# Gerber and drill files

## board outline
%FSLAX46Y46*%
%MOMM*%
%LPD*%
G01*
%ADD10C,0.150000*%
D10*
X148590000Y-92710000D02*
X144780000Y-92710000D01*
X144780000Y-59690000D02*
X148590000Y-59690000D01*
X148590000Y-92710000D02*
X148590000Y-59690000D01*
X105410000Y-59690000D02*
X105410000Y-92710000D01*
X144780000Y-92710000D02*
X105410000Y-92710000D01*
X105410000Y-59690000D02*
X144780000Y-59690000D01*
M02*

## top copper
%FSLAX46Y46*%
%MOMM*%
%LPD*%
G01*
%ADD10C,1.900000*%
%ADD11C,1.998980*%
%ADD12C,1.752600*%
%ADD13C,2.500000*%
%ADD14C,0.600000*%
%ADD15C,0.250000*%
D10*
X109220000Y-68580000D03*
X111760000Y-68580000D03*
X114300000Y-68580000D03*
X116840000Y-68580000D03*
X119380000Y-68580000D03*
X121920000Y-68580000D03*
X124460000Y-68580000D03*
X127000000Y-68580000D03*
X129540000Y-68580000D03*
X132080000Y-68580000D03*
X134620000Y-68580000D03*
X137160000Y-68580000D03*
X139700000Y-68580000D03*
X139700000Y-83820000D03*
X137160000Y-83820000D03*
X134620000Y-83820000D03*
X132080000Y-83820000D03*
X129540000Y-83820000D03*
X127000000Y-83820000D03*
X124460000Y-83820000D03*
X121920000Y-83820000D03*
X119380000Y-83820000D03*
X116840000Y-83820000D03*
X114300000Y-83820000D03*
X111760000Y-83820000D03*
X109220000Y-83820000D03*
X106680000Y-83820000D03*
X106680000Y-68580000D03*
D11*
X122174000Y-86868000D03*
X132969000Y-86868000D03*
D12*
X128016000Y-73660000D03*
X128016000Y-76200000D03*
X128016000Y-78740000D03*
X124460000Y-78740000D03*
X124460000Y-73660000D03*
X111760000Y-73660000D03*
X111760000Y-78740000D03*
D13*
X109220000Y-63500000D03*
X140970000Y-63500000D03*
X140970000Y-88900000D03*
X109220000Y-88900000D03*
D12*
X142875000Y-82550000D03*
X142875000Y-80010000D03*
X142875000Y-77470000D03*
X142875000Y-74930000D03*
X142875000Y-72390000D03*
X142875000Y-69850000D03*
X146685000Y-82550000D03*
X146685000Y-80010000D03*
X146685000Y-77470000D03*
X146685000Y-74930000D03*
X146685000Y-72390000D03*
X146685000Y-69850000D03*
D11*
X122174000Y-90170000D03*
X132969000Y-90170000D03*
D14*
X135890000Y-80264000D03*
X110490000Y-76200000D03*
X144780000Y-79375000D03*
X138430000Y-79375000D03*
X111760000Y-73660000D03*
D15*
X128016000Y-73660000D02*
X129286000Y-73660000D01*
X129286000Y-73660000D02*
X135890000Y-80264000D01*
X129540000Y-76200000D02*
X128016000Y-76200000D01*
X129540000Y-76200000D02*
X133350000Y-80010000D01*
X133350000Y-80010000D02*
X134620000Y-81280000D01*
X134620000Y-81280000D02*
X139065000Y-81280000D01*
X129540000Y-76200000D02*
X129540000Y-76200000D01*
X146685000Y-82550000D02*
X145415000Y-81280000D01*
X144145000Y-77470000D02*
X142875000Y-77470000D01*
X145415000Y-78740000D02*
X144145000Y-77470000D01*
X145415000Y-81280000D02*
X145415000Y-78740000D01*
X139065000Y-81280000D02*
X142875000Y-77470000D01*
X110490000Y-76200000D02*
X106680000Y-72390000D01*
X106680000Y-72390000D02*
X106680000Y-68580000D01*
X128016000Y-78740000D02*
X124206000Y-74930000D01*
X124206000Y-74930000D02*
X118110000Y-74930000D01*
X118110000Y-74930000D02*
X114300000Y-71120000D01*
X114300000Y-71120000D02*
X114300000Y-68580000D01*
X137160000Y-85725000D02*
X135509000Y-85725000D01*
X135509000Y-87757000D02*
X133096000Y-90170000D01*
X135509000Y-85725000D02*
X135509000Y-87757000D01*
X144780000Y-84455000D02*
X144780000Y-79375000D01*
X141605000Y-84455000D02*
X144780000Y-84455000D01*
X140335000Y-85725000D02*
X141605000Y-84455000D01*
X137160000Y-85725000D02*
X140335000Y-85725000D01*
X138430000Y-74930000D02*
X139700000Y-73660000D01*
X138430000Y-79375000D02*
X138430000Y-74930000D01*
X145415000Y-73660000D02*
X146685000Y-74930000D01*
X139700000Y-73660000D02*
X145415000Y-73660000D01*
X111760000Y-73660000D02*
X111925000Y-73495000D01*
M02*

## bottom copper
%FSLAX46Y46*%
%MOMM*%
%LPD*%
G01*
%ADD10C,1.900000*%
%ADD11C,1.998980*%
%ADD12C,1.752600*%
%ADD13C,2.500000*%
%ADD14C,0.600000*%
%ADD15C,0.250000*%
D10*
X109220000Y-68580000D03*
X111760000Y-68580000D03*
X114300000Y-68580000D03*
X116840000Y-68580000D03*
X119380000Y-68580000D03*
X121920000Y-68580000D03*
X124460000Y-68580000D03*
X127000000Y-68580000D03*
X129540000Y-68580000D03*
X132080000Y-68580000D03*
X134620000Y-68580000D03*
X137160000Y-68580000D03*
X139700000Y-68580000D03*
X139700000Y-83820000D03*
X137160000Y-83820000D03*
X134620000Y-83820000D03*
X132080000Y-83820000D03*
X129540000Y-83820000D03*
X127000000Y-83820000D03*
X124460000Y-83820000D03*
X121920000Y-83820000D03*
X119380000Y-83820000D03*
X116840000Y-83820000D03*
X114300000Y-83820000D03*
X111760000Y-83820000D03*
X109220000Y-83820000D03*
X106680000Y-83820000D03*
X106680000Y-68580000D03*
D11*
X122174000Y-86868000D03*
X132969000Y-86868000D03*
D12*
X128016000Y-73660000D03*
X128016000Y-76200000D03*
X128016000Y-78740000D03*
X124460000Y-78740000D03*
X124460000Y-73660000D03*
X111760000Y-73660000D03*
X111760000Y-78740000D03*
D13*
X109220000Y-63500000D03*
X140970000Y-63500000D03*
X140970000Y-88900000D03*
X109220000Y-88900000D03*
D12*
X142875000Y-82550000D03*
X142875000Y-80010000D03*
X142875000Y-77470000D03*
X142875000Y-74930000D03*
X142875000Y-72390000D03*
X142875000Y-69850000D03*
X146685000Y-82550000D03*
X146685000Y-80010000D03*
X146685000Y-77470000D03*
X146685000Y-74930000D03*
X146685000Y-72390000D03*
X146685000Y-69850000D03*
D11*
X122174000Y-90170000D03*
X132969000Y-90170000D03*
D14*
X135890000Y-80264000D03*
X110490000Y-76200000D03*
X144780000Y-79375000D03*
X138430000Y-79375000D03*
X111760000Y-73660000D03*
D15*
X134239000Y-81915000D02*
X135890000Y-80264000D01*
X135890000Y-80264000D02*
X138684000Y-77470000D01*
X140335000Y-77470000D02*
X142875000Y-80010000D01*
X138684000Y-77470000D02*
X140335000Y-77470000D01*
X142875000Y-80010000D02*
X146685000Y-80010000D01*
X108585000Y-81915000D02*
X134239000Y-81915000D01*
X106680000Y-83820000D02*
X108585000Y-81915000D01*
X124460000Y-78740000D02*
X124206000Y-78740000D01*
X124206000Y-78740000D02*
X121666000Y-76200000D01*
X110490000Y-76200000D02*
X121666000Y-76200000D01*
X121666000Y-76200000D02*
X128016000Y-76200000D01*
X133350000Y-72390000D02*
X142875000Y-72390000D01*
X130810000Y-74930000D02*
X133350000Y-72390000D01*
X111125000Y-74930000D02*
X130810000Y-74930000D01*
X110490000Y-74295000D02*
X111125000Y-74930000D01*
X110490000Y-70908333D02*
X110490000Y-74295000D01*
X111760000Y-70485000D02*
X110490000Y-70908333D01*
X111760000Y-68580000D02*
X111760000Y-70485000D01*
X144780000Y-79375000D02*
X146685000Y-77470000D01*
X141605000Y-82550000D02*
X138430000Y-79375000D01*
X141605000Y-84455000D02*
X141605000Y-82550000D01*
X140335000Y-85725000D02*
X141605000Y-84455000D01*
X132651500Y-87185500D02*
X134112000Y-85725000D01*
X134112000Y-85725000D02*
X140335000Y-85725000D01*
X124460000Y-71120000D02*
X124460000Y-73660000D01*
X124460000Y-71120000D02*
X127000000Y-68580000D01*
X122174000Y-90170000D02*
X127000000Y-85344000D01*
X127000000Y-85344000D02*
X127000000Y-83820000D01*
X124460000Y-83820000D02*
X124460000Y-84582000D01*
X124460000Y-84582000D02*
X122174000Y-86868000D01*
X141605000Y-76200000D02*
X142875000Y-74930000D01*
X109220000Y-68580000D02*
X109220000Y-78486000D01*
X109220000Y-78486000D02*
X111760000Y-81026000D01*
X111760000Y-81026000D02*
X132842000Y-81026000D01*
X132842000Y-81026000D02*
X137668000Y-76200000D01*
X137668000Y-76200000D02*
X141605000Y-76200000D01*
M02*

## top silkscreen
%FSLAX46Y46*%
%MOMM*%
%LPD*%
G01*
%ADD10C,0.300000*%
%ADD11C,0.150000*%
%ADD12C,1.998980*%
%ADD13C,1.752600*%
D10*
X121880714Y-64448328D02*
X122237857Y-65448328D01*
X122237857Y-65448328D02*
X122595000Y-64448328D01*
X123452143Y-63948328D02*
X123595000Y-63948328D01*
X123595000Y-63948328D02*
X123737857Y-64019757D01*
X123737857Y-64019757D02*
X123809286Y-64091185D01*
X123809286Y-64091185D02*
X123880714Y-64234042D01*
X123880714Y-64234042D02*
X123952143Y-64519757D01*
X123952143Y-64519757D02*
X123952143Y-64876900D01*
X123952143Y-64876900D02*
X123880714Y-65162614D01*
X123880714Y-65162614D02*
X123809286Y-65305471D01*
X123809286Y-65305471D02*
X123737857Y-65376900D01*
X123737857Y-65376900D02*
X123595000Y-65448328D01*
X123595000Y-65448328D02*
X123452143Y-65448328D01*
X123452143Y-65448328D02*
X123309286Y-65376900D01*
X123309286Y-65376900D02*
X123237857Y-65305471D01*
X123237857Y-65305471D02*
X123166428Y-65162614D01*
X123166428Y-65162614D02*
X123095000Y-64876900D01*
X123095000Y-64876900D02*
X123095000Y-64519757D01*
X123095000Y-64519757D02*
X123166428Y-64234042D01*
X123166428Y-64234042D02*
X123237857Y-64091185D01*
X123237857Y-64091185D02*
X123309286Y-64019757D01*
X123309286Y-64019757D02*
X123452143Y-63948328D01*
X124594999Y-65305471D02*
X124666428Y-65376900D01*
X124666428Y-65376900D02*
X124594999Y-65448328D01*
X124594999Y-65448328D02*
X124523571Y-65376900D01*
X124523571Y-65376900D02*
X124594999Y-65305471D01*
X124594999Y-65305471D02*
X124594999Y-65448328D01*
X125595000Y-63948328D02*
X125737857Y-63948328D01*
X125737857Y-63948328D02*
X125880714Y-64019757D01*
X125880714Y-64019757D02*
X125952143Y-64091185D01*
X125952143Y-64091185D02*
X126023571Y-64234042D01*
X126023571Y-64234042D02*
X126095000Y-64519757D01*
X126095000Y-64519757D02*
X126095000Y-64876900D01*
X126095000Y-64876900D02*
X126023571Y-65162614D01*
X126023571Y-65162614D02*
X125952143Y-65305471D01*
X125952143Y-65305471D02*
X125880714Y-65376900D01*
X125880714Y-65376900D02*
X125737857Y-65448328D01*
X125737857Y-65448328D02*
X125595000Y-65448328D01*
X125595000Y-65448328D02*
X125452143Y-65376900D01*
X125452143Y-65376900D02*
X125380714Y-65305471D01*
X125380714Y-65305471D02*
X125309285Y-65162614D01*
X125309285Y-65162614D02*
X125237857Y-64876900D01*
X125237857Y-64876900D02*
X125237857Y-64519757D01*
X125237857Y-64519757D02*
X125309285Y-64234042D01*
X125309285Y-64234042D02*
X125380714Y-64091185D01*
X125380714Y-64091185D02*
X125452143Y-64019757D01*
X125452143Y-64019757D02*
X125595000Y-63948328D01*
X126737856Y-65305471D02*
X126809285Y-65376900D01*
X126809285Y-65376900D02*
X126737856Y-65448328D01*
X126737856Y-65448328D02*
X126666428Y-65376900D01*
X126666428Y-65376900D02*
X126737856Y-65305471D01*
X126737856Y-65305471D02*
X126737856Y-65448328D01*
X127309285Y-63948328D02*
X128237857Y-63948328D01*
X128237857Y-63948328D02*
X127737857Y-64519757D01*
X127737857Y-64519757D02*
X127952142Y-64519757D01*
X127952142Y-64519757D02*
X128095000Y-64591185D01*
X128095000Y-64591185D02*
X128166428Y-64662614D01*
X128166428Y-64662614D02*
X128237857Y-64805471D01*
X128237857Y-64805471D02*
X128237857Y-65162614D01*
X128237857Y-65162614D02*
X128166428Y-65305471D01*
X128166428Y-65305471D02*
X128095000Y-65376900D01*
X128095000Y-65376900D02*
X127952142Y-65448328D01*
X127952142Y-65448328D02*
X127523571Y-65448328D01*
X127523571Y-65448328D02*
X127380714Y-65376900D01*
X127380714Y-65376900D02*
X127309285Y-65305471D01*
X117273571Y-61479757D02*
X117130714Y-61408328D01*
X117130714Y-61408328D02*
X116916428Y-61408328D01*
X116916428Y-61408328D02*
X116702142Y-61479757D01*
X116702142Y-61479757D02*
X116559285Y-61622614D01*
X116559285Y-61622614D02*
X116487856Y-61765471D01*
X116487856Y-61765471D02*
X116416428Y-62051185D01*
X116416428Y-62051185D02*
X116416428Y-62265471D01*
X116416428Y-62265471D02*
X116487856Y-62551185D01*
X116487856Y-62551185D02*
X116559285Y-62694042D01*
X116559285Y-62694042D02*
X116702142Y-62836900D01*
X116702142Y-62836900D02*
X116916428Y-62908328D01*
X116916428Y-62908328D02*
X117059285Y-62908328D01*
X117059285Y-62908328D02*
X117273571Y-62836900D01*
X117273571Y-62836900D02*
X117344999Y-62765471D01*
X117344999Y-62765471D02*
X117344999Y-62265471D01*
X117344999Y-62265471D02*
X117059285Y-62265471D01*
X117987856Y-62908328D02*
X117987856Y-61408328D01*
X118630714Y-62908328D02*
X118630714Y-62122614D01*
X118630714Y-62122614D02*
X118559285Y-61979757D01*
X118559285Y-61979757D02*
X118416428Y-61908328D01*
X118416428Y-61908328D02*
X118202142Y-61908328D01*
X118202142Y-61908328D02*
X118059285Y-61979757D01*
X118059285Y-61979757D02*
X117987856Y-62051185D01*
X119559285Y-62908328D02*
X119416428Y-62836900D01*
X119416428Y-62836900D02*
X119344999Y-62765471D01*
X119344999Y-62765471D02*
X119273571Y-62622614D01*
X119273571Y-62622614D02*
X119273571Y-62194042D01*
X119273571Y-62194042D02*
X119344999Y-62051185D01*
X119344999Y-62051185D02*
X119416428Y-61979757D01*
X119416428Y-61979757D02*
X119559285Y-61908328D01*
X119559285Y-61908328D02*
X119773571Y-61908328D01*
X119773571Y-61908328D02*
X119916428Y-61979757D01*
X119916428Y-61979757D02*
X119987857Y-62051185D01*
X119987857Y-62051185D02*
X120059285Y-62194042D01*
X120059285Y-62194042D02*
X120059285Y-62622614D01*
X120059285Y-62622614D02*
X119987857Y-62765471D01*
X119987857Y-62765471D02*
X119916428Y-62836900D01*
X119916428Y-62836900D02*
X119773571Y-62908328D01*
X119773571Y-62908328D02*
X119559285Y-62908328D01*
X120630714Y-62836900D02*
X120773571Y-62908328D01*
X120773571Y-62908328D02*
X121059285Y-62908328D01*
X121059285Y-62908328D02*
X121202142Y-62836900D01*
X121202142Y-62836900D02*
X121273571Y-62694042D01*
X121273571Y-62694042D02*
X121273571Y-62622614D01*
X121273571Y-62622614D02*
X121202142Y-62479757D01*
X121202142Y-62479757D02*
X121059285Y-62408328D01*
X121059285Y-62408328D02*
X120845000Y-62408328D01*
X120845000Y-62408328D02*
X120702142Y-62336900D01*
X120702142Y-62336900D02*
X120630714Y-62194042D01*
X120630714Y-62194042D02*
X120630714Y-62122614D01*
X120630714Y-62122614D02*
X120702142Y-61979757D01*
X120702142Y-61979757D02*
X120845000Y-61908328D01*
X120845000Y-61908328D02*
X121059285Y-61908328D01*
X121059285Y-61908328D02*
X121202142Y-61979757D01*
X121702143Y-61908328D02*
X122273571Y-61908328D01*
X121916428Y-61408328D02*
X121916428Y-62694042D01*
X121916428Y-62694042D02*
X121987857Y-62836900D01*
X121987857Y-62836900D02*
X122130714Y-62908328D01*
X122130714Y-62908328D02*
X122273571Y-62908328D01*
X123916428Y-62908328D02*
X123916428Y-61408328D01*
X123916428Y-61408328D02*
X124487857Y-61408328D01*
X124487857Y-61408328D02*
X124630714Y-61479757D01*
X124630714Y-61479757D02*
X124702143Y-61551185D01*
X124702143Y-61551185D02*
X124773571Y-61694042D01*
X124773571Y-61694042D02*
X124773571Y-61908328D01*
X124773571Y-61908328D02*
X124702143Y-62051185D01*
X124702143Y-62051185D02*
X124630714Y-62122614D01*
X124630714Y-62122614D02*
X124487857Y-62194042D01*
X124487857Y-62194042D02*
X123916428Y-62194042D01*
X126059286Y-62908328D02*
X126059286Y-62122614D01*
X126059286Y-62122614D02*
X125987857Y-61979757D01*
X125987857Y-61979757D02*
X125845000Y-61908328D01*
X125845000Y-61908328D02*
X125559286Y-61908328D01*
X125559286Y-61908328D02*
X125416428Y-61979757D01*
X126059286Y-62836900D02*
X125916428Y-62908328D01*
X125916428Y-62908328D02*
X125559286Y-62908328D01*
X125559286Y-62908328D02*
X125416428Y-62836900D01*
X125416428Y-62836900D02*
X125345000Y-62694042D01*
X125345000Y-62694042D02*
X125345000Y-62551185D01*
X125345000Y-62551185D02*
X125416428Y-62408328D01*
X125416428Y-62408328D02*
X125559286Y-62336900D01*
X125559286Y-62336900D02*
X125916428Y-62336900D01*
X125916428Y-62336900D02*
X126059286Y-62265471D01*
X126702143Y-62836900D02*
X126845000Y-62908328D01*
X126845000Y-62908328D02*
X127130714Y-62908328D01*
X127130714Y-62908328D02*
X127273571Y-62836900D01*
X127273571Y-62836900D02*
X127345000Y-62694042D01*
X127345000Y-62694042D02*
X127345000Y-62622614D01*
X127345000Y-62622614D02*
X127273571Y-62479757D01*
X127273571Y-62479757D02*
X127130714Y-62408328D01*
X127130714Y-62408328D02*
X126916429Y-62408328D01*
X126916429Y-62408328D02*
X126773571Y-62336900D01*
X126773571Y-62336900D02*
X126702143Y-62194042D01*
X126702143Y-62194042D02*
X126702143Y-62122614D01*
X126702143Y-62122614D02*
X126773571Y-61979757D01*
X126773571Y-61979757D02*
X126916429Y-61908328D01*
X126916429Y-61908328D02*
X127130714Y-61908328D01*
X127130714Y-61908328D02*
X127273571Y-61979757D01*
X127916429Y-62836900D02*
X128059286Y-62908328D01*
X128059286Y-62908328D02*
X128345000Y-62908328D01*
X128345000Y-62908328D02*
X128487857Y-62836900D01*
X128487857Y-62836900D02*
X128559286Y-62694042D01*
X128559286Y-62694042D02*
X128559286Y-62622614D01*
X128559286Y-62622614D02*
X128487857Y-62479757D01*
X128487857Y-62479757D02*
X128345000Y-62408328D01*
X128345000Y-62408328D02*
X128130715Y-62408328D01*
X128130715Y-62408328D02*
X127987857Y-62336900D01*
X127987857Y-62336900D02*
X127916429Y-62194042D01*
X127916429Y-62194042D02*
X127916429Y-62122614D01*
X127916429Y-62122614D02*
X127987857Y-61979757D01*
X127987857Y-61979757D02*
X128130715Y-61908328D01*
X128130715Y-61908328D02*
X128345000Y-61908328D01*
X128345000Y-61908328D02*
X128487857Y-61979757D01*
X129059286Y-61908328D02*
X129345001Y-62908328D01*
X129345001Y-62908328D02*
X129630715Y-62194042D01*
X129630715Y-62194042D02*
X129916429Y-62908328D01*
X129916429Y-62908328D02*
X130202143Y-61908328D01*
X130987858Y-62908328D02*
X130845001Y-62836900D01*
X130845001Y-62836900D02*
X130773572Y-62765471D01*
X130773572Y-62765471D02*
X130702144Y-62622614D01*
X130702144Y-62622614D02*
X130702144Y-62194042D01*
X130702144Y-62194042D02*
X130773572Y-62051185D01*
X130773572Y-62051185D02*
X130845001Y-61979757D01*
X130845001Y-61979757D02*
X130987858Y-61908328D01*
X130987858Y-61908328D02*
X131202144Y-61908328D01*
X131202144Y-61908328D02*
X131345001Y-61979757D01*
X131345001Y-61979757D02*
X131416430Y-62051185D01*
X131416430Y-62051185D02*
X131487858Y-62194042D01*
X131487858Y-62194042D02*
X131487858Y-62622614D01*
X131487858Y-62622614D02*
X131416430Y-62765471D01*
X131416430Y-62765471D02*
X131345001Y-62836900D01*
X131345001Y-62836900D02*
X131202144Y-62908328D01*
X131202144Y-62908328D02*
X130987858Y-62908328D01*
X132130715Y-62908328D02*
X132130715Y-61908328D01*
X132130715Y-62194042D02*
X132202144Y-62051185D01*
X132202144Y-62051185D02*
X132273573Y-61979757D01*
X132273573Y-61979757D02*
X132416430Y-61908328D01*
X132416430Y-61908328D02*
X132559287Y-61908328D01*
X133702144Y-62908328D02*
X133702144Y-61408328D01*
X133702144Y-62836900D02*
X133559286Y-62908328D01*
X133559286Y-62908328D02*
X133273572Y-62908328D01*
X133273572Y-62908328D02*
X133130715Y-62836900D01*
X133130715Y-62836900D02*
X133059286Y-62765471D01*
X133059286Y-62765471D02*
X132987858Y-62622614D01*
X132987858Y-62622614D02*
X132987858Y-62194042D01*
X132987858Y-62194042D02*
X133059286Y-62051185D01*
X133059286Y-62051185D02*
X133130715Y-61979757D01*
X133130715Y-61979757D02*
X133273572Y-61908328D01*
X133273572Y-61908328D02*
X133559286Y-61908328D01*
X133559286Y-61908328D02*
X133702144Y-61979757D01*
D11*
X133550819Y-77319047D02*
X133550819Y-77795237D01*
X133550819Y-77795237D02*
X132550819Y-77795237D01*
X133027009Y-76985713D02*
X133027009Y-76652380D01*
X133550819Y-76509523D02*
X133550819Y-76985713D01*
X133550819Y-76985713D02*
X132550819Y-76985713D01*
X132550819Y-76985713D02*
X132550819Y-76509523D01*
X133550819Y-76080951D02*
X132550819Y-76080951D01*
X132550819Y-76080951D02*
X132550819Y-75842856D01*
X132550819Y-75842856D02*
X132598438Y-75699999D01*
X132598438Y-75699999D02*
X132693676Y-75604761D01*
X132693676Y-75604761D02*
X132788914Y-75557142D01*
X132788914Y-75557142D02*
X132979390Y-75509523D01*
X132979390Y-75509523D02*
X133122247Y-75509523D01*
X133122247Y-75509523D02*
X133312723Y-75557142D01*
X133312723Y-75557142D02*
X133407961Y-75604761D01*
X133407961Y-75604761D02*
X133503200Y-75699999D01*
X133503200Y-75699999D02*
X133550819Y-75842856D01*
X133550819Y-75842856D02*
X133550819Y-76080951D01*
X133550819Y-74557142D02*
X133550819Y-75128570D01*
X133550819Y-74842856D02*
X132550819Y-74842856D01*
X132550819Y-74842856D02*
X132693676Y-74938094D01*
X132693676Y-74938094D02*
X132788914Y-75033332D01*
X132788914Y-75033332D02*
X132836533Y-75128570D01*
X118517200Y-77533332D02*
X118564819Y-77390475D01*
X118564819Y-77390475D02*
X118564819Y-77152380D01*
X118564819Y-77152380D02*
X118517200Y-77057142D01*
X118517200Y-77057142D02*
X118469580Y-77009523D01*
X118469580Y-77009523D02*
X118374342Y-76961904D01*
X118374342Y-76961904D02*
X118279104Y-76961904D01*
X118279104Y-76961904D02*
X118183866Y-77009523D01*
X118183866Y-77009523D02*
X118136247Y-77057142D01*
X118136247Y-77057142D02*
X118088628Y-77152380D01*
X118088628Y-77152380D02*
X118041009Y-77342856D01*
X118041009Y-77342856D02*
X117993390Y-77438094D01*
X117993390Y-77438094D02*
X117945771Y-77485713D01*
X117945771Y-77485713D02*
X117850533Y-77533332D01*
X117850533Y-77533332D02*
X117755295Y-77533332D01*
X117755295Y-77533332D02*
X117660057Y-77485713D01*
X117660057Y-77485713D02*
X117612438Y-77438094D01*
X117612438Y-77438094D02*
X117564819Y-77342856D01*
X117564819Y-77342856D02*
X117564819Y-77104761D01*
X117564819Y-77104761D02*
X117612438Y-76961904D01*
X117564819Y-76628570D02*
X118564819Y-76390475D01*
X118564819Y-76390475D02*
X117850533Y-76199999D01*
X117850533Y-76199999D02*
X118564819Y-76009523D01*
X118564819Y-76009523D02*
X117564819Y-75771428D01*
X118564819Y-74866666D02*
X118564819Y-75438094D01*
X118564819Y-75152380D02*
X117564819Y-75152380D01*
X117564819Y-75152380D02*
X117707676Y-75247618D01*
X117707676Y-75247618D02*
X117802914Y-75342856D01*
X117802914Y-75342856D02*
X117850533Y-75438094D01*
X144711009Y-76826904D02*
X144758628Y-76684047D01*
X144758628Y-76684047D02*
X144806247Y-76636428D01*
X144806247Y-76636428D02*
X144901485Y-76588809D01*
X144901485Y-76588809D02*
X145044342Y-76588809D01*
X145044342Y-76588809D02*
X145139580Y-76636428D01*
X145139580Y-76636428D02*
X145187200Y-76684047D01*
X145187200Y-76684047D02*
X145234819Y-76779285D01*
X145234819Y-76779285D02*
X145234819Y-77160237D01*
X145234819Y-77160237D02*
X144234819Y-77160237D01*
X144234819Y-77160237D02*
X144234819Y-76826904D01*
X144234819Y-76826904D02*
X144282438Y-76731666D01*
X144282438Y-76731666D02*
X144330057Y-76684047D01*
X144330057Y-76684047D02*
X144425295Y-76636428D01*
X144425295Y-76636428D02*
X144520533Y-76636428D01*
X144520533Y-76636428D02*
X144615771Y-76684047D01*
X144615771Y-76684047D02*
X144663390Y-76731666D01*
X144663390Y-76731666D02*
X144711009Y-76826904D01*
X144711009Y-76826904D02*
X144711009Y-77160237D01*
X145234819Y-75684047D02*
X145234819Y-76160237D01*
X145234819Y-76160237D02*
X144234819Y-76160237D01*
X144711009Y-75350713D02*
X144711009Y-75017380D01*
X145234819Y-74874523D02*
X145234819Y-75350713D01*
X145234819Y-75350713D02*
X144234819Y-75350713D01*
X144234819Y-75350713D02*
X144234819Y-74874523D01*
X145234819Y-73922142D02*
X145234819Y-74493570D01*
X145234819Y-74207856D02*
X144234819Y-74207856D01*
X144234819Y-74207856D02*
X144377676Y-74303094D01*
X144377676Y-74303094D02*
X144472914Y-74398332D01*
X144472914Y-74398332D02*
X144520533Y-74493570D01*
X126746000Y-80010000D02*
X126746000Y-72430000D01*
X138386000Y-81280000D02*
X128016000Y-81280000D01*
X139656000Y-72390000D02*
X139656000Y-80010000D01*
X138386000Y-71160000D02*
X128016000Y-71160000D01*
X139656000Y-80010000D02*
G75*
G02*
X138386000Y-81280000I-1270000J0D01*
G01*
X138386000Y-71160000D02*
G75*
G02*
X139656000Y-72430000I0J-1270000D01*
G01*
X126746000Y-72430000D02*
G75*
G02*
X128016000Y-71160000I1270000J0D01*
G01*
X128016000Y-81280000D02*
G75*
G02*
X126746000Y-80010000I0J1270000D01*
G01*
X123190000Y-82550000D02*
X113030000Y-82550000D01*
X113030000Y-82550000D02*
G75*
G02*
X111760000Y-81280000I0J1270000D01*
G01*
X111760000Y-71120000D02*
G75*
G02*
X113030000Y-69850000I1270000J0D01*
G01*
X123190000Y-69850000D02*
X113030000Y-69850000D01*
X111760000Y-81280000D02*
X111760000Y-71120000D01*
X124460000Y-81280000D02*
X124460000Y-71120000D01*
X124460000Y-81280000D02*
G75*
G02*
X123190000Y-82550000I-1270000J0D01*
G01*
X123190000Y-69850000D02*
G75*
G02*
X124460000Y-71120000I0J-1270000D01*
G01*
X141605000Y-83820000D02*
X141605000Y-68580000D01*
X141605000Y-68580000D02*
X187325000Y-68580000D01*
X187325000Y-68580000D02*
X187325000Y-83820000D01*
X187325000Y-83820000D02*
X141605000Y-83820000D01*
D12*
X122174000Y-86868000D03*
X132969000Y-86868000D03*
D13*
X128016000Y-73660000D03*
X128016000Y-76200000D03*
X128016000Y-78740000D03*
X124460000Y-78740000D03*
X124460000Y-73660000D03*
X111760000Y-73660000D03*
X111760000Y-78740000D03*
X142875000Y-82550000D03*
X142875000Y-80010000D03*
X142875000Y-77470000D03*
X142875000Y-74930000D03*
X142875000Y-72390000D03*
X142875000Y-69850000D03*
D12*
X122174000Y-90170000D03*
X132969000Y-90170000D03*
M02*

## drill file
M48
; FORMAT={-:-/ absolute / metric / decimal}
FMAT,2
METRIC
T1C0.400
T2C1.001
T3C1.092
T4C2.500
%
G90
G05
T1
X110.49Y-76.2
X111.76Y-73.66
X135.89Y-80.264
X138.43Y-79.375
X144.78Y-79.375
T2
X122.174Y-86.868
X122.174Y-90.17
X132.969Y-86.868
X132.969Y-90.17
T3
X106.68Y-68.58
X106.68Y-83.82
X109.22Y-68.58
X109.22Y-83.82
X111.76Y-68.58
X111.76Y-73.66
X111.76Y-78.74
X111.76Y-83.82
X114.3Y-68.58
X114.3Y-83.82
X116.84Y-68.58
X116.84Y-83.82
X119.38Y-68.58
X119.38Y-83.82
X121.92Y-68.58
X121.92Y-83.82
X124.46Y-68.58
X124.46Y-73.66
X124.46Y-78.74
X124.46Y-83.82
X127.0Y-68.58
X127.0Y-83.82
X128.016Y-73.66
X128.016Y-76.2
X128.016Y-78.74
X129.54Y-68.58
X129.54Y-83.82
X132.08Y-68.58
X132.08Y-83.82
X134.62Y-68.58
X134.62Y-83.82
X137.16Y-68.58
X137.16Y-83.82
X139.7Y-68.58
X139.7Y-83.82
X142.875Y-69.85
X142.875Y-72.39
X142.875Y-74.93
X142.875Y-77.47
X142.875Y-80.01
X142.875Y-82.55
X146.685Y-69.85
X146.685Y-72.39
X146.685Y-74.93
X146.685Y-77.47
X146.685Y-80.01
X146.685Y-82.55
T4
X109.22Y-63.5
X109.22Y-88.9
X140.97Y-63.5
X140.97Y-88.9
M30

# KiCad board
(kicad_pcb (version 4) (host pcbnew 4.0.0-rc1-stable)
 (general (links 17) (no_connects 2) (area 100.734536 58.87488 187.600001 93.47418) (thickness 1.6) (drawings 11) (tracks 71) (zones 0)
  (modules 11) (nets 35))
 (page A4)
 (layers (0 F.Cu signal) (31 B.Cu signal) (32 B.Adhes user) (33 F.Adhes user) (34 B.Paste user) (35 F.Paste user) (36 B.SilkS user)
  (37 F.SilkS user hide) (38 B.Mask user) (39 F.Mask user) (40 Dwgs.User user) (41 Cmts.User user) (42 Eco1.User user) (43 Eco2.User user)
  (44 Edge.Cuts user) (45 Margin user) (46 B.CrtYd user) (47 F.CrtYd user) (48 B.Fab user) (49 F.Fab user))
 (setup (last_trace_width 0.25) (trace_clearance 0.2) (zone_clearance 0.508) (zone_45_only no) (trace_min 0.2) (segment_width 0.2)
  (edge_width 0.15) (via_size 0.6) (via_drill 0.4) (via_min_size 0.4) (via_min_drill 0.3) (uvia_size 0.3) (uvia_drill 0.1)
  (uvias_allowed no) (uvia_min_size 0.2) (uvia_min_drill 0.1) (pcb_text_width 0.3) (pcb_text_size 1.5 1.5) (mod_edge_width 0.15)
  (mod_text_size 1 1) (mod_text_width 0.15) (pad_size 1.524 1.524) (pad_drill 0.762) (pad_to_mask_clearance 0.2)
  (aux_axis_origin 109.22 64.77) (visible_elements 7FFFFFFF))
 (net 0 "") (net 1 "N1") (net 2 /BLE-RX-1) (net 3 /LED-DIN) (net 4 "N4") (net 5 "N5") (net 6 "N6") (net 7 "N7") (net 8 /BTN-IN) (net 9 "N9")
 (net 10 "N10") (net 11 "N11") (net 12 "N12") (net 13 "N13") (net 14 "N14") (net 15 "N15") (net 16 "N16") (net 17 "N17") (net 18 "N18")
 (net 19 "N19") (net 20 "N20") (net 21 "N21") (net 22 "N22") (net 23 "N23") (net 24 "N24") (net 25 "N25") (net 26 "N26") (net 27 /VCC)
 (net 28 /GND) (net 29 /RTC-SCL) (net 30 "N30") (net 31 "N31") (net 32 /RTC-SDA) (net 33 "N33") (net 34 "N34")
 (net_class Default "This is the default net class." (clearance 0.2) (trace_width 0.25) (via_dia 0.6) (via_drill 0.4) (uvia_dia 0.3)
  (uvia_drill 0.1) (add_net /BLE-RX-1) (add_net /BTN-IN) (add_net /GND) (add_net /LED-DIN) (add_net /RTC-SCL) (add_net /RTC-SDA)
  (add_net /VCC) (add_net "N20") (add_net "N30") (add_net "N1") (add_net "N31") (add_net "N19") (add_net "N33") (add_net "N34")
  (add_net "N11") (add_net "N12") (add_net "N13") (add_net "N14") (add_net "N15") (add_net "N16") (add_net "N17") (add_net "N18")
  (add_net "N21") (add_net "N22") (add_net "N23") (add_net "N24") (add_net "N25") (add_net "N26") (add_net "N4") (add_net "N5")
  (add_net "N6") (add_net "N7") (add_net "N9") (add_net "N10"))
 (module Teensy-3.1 (layer B.Cu) (at 109.22 68.58)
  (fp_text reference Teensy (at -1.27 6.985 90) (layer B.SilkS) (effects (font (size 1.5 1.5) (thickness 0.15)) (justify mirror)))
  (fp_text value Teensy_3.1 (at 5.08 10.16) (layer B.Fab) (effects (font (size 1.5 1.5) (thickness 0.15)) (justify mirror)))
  (pad 0 thru_hole circle (at 0 0) (size 1.9 1.9) (drill 1.0922) (layers *.Cu *.Mask B.SilkS) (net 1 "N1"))
  (pad 1 thru_hole circle (at 2.54 0) (size 1.9 1.9) (drill 1.0922) (layers *.Cu *.Mask B.SilkS) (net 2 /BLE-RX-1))
  (pad 2 thru_hole circle (at 5.08 0) (size 1.9 1.9) (drill 1.0922) (layers *.Cu *.Mask B.SilkS) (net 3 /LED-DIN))
  (pad 3 thru_hole circle (at 7.62 0) (size 1.9 1.9) (drill 1.0922) (layers *.Cu *.Mask B.SilkS) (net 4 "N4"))
  (pad 4 thru_hole circle (at 10.16 0) (size 1.9 1.9) (drill 1.0922) (layers *.Cu *.Mask B.SilkS) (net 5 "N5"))
  (pad 5 thru_hole circle (at 12.7 0) (size 1.9 1.9) (drill 1.0922) (layers *.Cu *.Mask B.SilkS) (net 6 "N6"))
  (pad 6 thru_hole circle (at 15.24 0) (size 1.9 1.9) (drill 1.0922) (layers *.Cu *.Mask B.SilkS) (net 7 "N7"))
  (pad 7 thru_hole circle (at 17.78 0) (size 1.9 1.9) (drill 1.0922) (layers *.Cu *.Mask B.SilkS) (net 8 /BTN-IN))
  (pad 8 thru_hole circle (at 20.32 0) (size 1.9 1.9) (drill 1.0922) (layers *.Cu *.Mask B.SilkS) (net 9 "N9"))
  (pad 9 thru_hole circle (at 22.86 0) (size 1.9 1.9) (drill 1.0922) (layers *.Cu *.Mask B.SilkS) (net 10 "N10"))
  (pad 10 thru_hole circle (at 25.4 0) (size 1.9 1.9) (drill 1.0922) (layers *.Cu *.Mask B.SilkS) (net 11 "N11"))
  (pad 11 thru_hole circle (at 27.94 0) (size 1.9 1.9) (drill 1.0922) (layers *.Cu *.Mask B.SilkS) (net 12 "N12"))
  (pad 12 thru_hole circle (at 30.48 0) (size 1.9 1.9) (drill 1.0922) (layers *.Cu *.Mask B.SilkS) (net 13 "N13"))
  (pad 13 thru_hole circle (at 30.48 15.24) (size 1.9 1.9) (drill 1.0922) (layers *.Cu *.Mask B.SilkS) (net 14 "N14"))
  (pad 14 thru_hole circle (at 27.94 15.24) (size 1.9 1.9) (drill 1.0922) (layers *.Cu *.Mask B.SilkS) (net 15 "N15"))
  (pad 15 thru_hole circle (at 25.4 15.24) (size 1.9 1.9) (drill 1.0922) (layers *.Cu *.Mask B.SilkS) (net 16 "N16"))
  (pad 16 thru_hole circle (at 22.86 15.24) (size 1.9 1.9) (drill 1.0922) (layers *.Cu *.Mask B.SilkS) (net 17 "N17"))
  (pad 17 thru_hole circle (at 20.32 15.24) (size 1.9 1.9) (drill 1.0922) (layers *.Cu *.Mask B.SilkS) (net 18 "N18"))
  (pad 18 thru_hole circle (at 17.78 15.24) (size 1.9 1.9) (drill 1.0922) (layers *.Cu *.Mask B.SilkS) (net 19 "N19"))
  (pad 19 thru_hole circle (at 15.24 15.24) (size 1.9 1.9) (drill 1.0922) (layers *.Cu *.Mask B.SilkS) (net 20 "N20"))
  (pad 20 thru_hole circle (at 12.7 15.24) (size 1.9 1.9) (drill 1.0922) (layers *.Cu *.Mask B.SilkS) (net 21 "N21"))
  (pad 21 thru_hole circle (at 10.16 15.24) (size 1.9 1.9) (drill 1.0922) (layers *.Cu *.Mask B.SilkS) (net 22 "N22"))
  (pad 22 thru_hole circle (at 7.62 15.24) (size 1.9 1.9) (drill 1.0922) (layers *.Cu *.Mask B.SilkS) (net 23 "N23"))
  (pad 23 thru_hole circle (at 5.08 15.24) (size 1.9 1.9) (drill 1.0922) (layers *.Cu *.Mask B.SilkS) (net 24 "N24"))
  (pad 24 thru_hole circle (at 2.54 15.24) (size 1.9 1.9) (drill 1.0922) (layers *.Cu *.Mask B.SilkS) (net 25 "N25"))
  (pad 25 thru_hole circle (at 0 15.24) (size 1.9 1.9) (drill 1.0922) (layers *.Cu *.Mask B.SilkS) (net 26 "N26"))
  (pad 26 thru_hole circle (at -2.54 15.24) (size 1.9 1.9) (drill 1.0922) (layers *.Cu *.Mask B.SilkS) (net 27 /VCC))
  (pad 27 thru_hole circle (at -2.54 0) (size 1.9 1.9) (drill 1.0922) (layers *.Cu *.Mask B.SilkS) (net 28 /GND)))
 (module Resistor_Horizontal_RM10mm (layer B.Cu) (at 127.254 86.868)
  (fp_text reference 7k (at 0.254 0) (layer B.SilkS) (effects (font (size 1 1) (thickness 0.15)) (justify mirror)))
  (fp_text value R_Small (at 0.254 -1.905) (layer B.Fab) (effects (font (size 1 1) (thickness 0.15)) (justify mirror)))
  (pad 1 thru_hole circle (at -5.08 0) (size 1.99898 1.99898) (drill 1.00076) (layers *.Cu *.SilkS *.Mask) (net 20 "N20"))
  (pad 2 thru_hole circle (at 5.715 0) (size 1.99898 1.99898) (drill 1.00076) (layers *.Cu *.SilkS *.Mask) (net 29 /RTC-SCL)))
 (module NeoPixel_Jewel (layer F.Cu) (at 126.746 81.28 90)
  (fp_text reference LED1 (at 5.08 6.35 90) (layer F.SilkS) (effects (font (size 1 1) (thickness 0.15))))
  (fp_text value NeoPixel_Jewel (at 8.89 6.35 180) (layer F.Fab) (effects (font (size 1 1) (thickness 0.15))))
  (fp_line (start 1.27 0) (end 8.85 0) (layer F.SilkS) (width 0.15))
  (fp_line (start 0 11.64) (end 0 1.27) (layer F.SilkS) (width 0.15))
  (fp_line (start 8.89 12.91) (end 1.27 12.91) (layer F.SilkS) (width 0.15))
  (fp_line (start 10.12 11.64) (end 10.12 1.27) (layer F.SilkS) (width 0.15))
  (fp_arc (start 1.27 11.64) (end 1.27 12.91) (angle 90) (layer F.SilkS) (width 0.15))
  (fp_arc (start 8.85 11.64) (end 10.12 11.64) (angle 90) (layer F.SilkS) (width 0.15))
  (fp_arc (start 8.85 1.27) (end 8.85 0) (angle 90) (layer F.SilkS) (width 0.15))
  (fp_arc (start 1.27 1.27) (end 0 1.27) (angle 90) (layer F.SilkS) (width 0.15))
  (pad 1 thru_hole circle (at 7.62 1.27 90) (size 1.7526 1.7526) (drill 1.0922) (layers *.Cu *.Mask F.SilkS) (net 27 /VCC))
  (pad 2 thru_hole circle (at 5.08 1.27 90) (size 1.7526 1.7526) (drill 1.0922) (layers *.Cu *.Mask F.SilkS) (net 28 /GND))
  (pad 3 thru_hole circle (at 2.54 1.27 90) (size 1.7526 1.7526) (drill 1.0922) (layers *.Cu *.Mask F.SilkS) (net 3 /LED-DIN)))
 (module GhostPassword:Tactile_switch (layer F.Cu) (at 118.11 76.2 270)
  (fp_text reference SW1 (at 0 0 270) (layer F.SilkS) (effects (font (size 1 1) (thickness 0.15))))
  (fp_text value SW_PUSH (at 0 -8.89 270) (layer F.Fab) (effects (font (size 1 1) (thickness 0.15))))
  (fp_line (start 6.35 -5.08) (end 6.35 5.08) (layer F.SilkS) (width 0.15))
  (fp_arc (start 5.08 5.08) (end 6.35 5.08) (angle 90) (layer F.SilkS) (width 0.15))
  (fp_arc (start -5.08 5.08) (end -5.08 6.35) (angle 90) (layer F.SilkS) (width 0.15))
  (fp_line (start -6.35 -5.08) (end -6.35 5.08) (layer F.SilkS) (width 0.15))
  (fp_line (start 5.08 6.35) (end -5.08 6.35) (layer F.SilkS) (width 0.15))
  (fp_line (start 5.08 -6.35) (end -5.08 -6.35) (layer F.SilkS) (width 0.15))
  (fp_arc (start 5.08 -5.08) (end 5.08 -6.35) (angle 90) (layer F.SilkS) (width 0.15))
  (fp_arc (start -5.08 -5.08) (end -6.35 -5.08) (angle 90) (layer F.SilkS) (width 0.15))
  (pad 2 thru_hole circle (at 2.54 -6.35 270) (size 1.7526 1.7526) (drill 1.0922) (layers *.Cu *.Mask F.SilkS) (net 28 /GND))
  (pad 1 thru_hole circle (at -2.54 -6.35 270) (size 1.7526 1.7526) (drill 1.0922) (layers *.Cu *.Mask F.SilkS) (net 8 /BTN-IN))
  (pad 1 thru_hole circle (at -2.54 6.35 270) (size 1.7526 1.7526) (drill 1.0922) (layers *.Cu *.Mask F.SilkS) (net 8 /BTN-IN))
  (pad 2 thru_hole circle (at 2.54 6.35 270) (size 1.7526 1.7526) (drill 1.0922) (layers *.Cu *.Mask F.SilkS) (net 28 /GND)))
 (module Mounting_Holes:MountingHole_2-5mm (layer F.Cu) (at 109.22 63.5)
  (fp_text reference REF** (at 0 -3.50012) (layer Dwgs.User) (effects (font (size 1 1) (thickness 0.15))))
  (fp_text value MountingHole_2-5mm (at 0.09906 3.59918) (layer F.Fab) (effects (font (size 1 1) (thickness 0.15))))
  (pad 1 thru_hole circle (at 0 0) (size 2.5 2.5) (drill 2.5) (layers)))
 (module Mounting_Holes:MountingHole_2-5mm (layer F.Cu) (at 140.97 63.5)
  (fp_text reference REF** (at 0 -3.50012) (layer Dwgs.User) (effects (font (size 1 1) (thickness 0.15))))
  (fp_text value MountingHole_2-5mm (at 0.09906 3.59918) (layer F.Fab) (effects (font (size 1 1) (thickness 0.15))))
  (pad 1 thru_hole circle (at 0 0) (size 2.5 2.5) (drill 2.5) (layers)))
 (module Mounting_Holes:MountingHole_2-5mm (layer F.Cu) (at 140.97 88.9)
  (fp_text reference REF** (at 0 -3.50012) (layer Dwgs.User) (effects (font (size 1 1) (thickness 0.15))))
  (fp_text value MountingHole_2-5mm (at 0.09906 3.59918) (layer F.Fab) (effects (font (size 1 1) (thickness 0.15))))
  (pad 1 thru_hole circle (at 0 0) (size 2.5 2.5) (drill 2.5) (layers)))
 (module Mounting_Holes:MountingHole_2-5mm (layer F.Cu) (at 109.22 88.9)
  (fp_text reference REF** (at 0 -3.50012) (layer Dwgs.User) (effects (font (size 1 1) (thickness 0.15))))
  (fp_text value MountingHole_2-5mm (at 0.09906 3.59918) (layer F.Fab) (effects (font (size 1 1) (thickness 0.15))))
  (pad 1 thru_hole circle (at 0 0) (size 2.5 2.5) (drill 2.5) (layers)))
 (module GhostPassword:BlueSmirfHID (layer F.Cu) (at 141.605 83.82 90)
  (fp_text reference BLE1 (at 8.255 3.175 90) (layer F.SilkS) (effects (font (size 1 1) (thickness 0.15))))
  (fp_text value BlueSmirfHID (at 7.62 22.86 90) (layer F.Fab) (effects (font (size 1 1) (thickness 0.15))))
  (fp_line (start 0 0) (end 15.24 0) (layer F.SilkS) (width 0.15))
  (fp_line (start 15.24 0) (end 15.24 45.72) (layer F.SilkS) (width 0.15))
  (fp_line (start 15.24 45.72) (end 0 45.72) (layer F.SilkS) (width 0.15))
  (fp_line (start 0 45.72) (end 0 0) (layer F.SilkS) (width 0.15))
  (pad 1 thru_hole circle (at 1.27 1.27 90) (size 1.7526 1.7526) (drill 1.0922) (layers *.Cu *.Mask F.SilkS) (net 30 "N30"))
  (pad 2 thru_hole circle (at 3.81 1.27 90) (size 1.7526 1.7526) (drill 1.0922) (layers *.Cu *.Mask F.SilkS) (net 27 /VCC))
  (pad 3 thru_hole circle (at 6.35 1.27 90) (size 1.7526 1.7526) (drill 1.0922) (layers *.Cu *.Mask F.SilkS) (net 28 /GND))
  (pad 4 thru_hole circle (at 8.89 1.27 90) (size 1.7526 1.7526) (drill 1.0922) (layers *.Cu *.Mask F.SilkS) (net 1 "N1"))
  (pad 5 thru_hole circle (at 11.43 1.27 90) (size 1.7526 1.7526) (drill 1.0922) (layers *.Cu *.Mask F.SilkS) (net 2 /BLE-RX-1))
  (pad 6 thru_hole circle (at 13.97 1.27 90) (size 1.7526 1.7526) (drill 1.0922) (layers *.Cu *.Mask F.SilkS) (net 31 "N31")))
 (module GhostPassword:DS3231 (layer B.Cu) (at 144.145 64.77 270)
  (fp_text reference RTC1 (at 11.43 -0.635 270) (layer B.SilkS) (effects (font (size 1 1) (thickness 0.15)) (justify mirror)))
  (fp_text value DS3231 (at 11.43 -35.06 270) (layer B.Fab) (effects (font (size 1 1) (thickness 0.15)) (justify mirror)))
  (pad 1 thru_hole circle (at 17.78 -2.54 270) (size 1.7526 1.7526) (drill 1.0922) (layers *.Cu *.Mask B.SilkS) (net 28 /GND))
  (pad 2 thru_hole circle (at 15.24 -2.54 270) (size 1.7526 1.7526) (drill 1.0922) (layers *.Cu *.Mask B.SilkS) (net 27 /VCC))
  (pad 3 thru_hole circle (at 12.7 -2.54 270) (size 1.7526 1.7526) (drill 1.0922) (layers *.Cu *.Mask B.SilkS) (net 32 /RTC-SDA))
  (pad 4 thru_hole circle (at 10.16 -2.54 270) (size 1.7526 1.7526) (drill 1.0922) (layers *.Cu *.Mask B.SilkS) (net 29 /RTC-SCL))
  (pad 5 thru_hole circle (at 7.62 -2.54 270) (size 1.7526 1.7526) (drill 1.0922) (layers *.Cu *.Mask B.SilkS) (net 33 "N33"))
  (pad 6 thru_hole circle (at 5.08 -2.54 270) (size 1.7526 1.7526) (drill 1.0922) (layers *.Cu *.Mask B.SilkS) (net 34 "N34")))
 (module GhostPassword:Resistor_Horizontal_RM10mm (layer B.Cu) (at 127.254 90.17)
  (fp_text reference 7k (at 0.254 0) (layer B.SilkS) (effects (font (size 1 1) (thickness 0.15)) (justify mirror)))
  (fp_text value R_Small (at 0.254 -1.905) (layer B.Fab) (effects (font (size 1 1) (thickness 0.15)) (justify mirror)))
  (pad 1 thru_hole circle (at -5.08 0) (size 1.99898 1.99898) (drill 1.00076) (layers *.Cu *.SilkS *.Mask) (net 19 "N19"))
  (pad 2 thru_hole circle (at 5.715 0) (size 1.99898 1.99898) (drill 1.00076) (layers *.Cu *.SilkS *.Mask) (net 32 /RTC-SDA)))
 (gr_line (start 148.59 92.71) (end 144.78 92.71) (angle 90) (layer Edge.Cuts) (width 0.15))
 (gr_line (start 144.78 59.69) (end 148.59 59.69) (angle 90) (layer Edge.Cuts) (width 0.15))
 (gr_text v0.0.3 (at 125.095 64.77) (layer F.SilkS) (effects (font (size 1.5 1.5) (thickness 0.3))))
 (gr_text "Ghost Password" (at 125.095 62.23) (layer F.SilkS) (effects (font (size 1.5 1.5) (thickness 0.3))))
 (gr_line (start 148.59 92.71) (end 148.59 59.69) (angle 90) (layer Edge.Cuts) (width 0.15))
 (gr_line (start 105.41 59.69) (end 105.41 92.71) (angle 90) (layer Edge.Cuts) (width 0.15))
 (gr_line (start 144.78 92.71) (end 105.41 92.71) (angle 90) (layer Edge.Cuts) (width 0.15))
 (gr_line (start 105.41 59.69) (end 144.78 59.69) (angle 90) (layer Edge.Cuts) (width 0.15))
 (segment (start 128.016 73.66) (end 129.286 73.66) (width 0.25) (layer F.Cu) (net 27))
 (via (at 135.89 80.264) (size 0.6) (drill 0.4) (layers F.Cu B.Cu) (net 27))
 (segment (start 129.286 73.66) (end 135.89 80.264) (width 0.25) (layer F.Cu) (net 27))
 (segment (start 134.239 81.915) (end 135.89 80.264) (width 0.25) (layer B.Cu) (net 27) (status 20))
 (segment (start 135.89 80.264) (end 138.684 77.47) (width 0.25) (layer B.Cu) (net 27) (status 20))
 (segment (start 140.335 77.47) (end 142.875 80.01) (width 0.25) (layer B.Cu) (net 27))
 (segment (start 138.684 77.47) (end 140.335 77.47) (width 0.25) (layer B.Cu) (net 27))
 (segment (start 142.875 80.01) (end 146.685 80.01) (width 0.25) (layer B.Cu) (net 27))
 (segment (start 108.585 81.915) (end 134.239 81.915) (width 0.25) (layer B.Cu) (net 27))
 (segment (start 106.68 83.82) (end 108.585 81.915) (width 0.25) (layer B.Cu) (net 27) (status 10))
 (segment (start 129.54 76.2) (end 128.016 76.2) (width 0.25) (layer F.Cu) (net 28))
 (segment (start 124.46 78.74) (end 124.206 78.74) (width 0.25) (layer B.Cu) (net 28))
 (segment (start 124.206 78.74) (end 121.666 76.2) (width 0.25) (layer B.Cu) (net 28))
 (segment (start 110.49 76.2) (end 121.666 76.2) (width 0.25) (layer B.Cu) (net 28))
 (segment (start 121.666 76.2) (end 128.016 76.2) (width 0.25) (layer B.Cu) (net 28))
 (via (at 110.49 76.2) (size 0.6) (drill 0.4) (layers F.Cu B.Cu) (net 28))
 (segment (start 129.54 76.2) (end 133.35 80.01) (width 0.25) (layer F.Cu) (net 28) (status 10))
 (segment (start 133.35 80.01) (end 134.62 81.28) (width 0.25) (layer F.Cu) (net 28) (status 10))
 (segment (start 134.62 81.28) (end 139.065 81.28) (width 0.25) (layer F.Cu) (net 28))
 (segment (start 129.54 76.2) (end 129.54 76.2) (width 0.25) (layer F.Cu) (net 28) (status 10))
 (segment (start 146.685 82.55) (end 145.415 81.28) (width 0.25) (layer F.Cu) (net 28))
 (segment (start 144.145 77.47) (end 142.875 77.47) (width 0.25) (layer F.Cu) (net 28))
 (segment (start 145.415 78.74) (end 144.145 77.47) (width 0.25) (layer F.Cu) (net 28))
 (segment (start 145.415 81.28) (end 145.415 78.74) (width 0.25) (layer F.Cu) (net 28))
 (segment (start 139.065 81.28) (end 142.875 77.47) (width 0.25) (layer F.Cu) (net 28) (status 20))
 (segment (start 110.49 76.2) (end 106.68 72.39) (width 0.25) (layer F.Cu) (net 28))
 (segment (start 106.68 72.39) (end 106.68 68.58) (width 0.25) (layer F.Cu) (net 28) (status 20))
 (segment (start 133.35 72.39) (end 142.875 72.39) (width 0.25) (layer B.Cu) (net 2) (status 20))
 (segment (start 130.81 74.93) (end 133.35 72.39) (width 0.25) (layer B.Cu) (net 2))
 (segment (start 111.125 74.93) (end 130.81 74.93) (width 0.25) (layer B.Cu) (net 2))
 (segment (start 110.49 74.295) (end 111.125 74.93) (width 0.25) (layer B.Cu) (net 2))
 (segment (start 110.49 70.908333) (end 110.49 74.295) (width 0.25) (layer B.Cu) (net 2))
 (segment (start 111.76 70.485) (end 110.49 70.908333) (width 0.25) (layer B.Cu) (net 2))
 (segment (start 111.76 68.58) (end 111.76 70.485) (width 0.25) (layer B.Cu) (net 2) (status 10))
 (segment (start 128.016 78.74) (end 124.206 74.93) (width 0.25) (layer F.Cu) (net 3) (status 10))
 (segment (start 124.206 74.93) (end 118.11 74.93) (width 0.25) (layer F.Cu) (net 3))
 (segment (start 118.11 74.93) (end 114.3 71.12) (width 0.25) (layer F.Cu) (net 3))
 (segment (start 114.3 71.12) (end 114.3 68.58) (width 0.25) (layer F.Cu) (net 3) (status 20))
 (segment (start 137.16 85.725) (end 135.509 85.725) (width 0.25) (layer F.Cu) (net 32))
 (segment (start 135.509 87.757) (end 133.096 90.17) (width 0.25) (layer F.Cu) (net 32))
 (segment (start 135.509 85.725) (end 135.509 87.757) (width 0.25) (layer F.Cu) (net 32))
 (segment (start 144.78 79.375) (end 146.685 77.47) (width 0.25) (layer B.Cu) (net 32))
 (via (at 144.78 79.375) (size 0.6) (drill 0.4) (layers F.Cu B.Cu) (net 32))
 (segment (start 144.78 84.455) (end 144.78 79.375) (width 0.25) (layer F.Cu) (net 32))
 (segment (start 141.605 84.455) (end 144.78 84.455) (width 0.25) (layer F.Cu) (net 32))
 (segment (start 140.335 85.725) (end 141.605 84.455) (width 0.25) (layer F.Cu) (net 32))
 (segment (start 137.16 85.725) (end 140.335 85.725) (width 0.25) (layer F.Cu) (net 32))
 (segment (start 138.43 74.93) (end 139.7 73.66) (width 0.25) (layer F.Cu) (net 29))
 (segment (start 138.43 79.375) (end 138.43 74.93) (width 0.25) (layer F.Cu) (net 29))
 (via (at 138.43 79.375) (size 0.6) (drill 0.4) (layers F.Cu B.Cu) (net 29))
 (segment (start 141.605 82.55) (end 138.43 79.375) (width 0.25) (layer B.Cu) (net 29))
 (segment (start 141.605 84.455) (end 141.605 82.55) (width 0.25) (layer B.Cu) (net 29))
 (segment (start 140.335 85.725) (end 141.605 84.455) (width 0.25) (layer B.Cu) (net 29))
 (segment (start 132.6515 87.1855) (end 134.112 85.725) (width 0.25) (layer B.Cu) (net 29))
 (segment (start 145.415 73.66) (end 146.685 74.93) (width 0.25) (layer F.Cu) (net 29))
 (segment (start 139.7 73.66) (end 145.415 73.66) (width 0.25) (layer F.Cu) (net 29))
 (segment (start 134.112 85.725) (end 140.335 85.725) (width 0.25) (layer B.Cu) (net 29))
 (segment (start 111.76 73.66) (end 111.925 73.495) (width 0.25) (layer F.Cu) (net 8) (status 30))
 (via (at 111.76 73.66) (size 0.6) (drill 0.4) (layers F.Cu B.Cu) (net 8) (status 30))
 (segment (start 124.46 71.12) (end 124.46 73.66) (width 0.25) (layer B.Cu) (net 8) (status 20))
 (segment (start 124.46 71.12) (end 127 68.58) (width 0.25) (layer B.Cu) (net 8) (status 10))
 (segment (start 122.174 90.17) (end 127 85.344) (width 0.25) (layer B.Cu) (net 19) (status 400000))
 (segment (start 127 85.344) (end 127 83.82) (width 0.25) (layer B.Cu) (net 19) (status 800000))
 (segment (start 124.46 83.82) (end 124.46 84.582) (width 0.25) (layer B.Cu) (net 20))
 (segment (start 124.46 84.582) (end 122.174 86.868) (width 0.25) (layer B.Cu) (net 20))
 (segment (start 141.605 76.2) (end 142.875 74.93) (width 0.25) (layer B.Cu) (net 1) (status 20))
 (segment (start 109.22 68.58) (end 109.22 78.486) (width 0.25) (layer B.Cu) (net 1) (status 10))
 (segment (start 109.22 78.486) (end 111.76 81.026) (width 0.25) (layer B.Cu) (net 1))
 (segment (start 111.76 81.026) (end 132.842 81.026) (width 0.25) (layer B.Cu) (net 1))
 (segment (start 132.842 81.026) (end 137.668 76.2) (width 0.25) (layer B.Cu) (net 1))
 (segment (start 137.668 76.2) (end 141.605 76.2) (width 0.25) (layer B.Cu) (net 1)))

